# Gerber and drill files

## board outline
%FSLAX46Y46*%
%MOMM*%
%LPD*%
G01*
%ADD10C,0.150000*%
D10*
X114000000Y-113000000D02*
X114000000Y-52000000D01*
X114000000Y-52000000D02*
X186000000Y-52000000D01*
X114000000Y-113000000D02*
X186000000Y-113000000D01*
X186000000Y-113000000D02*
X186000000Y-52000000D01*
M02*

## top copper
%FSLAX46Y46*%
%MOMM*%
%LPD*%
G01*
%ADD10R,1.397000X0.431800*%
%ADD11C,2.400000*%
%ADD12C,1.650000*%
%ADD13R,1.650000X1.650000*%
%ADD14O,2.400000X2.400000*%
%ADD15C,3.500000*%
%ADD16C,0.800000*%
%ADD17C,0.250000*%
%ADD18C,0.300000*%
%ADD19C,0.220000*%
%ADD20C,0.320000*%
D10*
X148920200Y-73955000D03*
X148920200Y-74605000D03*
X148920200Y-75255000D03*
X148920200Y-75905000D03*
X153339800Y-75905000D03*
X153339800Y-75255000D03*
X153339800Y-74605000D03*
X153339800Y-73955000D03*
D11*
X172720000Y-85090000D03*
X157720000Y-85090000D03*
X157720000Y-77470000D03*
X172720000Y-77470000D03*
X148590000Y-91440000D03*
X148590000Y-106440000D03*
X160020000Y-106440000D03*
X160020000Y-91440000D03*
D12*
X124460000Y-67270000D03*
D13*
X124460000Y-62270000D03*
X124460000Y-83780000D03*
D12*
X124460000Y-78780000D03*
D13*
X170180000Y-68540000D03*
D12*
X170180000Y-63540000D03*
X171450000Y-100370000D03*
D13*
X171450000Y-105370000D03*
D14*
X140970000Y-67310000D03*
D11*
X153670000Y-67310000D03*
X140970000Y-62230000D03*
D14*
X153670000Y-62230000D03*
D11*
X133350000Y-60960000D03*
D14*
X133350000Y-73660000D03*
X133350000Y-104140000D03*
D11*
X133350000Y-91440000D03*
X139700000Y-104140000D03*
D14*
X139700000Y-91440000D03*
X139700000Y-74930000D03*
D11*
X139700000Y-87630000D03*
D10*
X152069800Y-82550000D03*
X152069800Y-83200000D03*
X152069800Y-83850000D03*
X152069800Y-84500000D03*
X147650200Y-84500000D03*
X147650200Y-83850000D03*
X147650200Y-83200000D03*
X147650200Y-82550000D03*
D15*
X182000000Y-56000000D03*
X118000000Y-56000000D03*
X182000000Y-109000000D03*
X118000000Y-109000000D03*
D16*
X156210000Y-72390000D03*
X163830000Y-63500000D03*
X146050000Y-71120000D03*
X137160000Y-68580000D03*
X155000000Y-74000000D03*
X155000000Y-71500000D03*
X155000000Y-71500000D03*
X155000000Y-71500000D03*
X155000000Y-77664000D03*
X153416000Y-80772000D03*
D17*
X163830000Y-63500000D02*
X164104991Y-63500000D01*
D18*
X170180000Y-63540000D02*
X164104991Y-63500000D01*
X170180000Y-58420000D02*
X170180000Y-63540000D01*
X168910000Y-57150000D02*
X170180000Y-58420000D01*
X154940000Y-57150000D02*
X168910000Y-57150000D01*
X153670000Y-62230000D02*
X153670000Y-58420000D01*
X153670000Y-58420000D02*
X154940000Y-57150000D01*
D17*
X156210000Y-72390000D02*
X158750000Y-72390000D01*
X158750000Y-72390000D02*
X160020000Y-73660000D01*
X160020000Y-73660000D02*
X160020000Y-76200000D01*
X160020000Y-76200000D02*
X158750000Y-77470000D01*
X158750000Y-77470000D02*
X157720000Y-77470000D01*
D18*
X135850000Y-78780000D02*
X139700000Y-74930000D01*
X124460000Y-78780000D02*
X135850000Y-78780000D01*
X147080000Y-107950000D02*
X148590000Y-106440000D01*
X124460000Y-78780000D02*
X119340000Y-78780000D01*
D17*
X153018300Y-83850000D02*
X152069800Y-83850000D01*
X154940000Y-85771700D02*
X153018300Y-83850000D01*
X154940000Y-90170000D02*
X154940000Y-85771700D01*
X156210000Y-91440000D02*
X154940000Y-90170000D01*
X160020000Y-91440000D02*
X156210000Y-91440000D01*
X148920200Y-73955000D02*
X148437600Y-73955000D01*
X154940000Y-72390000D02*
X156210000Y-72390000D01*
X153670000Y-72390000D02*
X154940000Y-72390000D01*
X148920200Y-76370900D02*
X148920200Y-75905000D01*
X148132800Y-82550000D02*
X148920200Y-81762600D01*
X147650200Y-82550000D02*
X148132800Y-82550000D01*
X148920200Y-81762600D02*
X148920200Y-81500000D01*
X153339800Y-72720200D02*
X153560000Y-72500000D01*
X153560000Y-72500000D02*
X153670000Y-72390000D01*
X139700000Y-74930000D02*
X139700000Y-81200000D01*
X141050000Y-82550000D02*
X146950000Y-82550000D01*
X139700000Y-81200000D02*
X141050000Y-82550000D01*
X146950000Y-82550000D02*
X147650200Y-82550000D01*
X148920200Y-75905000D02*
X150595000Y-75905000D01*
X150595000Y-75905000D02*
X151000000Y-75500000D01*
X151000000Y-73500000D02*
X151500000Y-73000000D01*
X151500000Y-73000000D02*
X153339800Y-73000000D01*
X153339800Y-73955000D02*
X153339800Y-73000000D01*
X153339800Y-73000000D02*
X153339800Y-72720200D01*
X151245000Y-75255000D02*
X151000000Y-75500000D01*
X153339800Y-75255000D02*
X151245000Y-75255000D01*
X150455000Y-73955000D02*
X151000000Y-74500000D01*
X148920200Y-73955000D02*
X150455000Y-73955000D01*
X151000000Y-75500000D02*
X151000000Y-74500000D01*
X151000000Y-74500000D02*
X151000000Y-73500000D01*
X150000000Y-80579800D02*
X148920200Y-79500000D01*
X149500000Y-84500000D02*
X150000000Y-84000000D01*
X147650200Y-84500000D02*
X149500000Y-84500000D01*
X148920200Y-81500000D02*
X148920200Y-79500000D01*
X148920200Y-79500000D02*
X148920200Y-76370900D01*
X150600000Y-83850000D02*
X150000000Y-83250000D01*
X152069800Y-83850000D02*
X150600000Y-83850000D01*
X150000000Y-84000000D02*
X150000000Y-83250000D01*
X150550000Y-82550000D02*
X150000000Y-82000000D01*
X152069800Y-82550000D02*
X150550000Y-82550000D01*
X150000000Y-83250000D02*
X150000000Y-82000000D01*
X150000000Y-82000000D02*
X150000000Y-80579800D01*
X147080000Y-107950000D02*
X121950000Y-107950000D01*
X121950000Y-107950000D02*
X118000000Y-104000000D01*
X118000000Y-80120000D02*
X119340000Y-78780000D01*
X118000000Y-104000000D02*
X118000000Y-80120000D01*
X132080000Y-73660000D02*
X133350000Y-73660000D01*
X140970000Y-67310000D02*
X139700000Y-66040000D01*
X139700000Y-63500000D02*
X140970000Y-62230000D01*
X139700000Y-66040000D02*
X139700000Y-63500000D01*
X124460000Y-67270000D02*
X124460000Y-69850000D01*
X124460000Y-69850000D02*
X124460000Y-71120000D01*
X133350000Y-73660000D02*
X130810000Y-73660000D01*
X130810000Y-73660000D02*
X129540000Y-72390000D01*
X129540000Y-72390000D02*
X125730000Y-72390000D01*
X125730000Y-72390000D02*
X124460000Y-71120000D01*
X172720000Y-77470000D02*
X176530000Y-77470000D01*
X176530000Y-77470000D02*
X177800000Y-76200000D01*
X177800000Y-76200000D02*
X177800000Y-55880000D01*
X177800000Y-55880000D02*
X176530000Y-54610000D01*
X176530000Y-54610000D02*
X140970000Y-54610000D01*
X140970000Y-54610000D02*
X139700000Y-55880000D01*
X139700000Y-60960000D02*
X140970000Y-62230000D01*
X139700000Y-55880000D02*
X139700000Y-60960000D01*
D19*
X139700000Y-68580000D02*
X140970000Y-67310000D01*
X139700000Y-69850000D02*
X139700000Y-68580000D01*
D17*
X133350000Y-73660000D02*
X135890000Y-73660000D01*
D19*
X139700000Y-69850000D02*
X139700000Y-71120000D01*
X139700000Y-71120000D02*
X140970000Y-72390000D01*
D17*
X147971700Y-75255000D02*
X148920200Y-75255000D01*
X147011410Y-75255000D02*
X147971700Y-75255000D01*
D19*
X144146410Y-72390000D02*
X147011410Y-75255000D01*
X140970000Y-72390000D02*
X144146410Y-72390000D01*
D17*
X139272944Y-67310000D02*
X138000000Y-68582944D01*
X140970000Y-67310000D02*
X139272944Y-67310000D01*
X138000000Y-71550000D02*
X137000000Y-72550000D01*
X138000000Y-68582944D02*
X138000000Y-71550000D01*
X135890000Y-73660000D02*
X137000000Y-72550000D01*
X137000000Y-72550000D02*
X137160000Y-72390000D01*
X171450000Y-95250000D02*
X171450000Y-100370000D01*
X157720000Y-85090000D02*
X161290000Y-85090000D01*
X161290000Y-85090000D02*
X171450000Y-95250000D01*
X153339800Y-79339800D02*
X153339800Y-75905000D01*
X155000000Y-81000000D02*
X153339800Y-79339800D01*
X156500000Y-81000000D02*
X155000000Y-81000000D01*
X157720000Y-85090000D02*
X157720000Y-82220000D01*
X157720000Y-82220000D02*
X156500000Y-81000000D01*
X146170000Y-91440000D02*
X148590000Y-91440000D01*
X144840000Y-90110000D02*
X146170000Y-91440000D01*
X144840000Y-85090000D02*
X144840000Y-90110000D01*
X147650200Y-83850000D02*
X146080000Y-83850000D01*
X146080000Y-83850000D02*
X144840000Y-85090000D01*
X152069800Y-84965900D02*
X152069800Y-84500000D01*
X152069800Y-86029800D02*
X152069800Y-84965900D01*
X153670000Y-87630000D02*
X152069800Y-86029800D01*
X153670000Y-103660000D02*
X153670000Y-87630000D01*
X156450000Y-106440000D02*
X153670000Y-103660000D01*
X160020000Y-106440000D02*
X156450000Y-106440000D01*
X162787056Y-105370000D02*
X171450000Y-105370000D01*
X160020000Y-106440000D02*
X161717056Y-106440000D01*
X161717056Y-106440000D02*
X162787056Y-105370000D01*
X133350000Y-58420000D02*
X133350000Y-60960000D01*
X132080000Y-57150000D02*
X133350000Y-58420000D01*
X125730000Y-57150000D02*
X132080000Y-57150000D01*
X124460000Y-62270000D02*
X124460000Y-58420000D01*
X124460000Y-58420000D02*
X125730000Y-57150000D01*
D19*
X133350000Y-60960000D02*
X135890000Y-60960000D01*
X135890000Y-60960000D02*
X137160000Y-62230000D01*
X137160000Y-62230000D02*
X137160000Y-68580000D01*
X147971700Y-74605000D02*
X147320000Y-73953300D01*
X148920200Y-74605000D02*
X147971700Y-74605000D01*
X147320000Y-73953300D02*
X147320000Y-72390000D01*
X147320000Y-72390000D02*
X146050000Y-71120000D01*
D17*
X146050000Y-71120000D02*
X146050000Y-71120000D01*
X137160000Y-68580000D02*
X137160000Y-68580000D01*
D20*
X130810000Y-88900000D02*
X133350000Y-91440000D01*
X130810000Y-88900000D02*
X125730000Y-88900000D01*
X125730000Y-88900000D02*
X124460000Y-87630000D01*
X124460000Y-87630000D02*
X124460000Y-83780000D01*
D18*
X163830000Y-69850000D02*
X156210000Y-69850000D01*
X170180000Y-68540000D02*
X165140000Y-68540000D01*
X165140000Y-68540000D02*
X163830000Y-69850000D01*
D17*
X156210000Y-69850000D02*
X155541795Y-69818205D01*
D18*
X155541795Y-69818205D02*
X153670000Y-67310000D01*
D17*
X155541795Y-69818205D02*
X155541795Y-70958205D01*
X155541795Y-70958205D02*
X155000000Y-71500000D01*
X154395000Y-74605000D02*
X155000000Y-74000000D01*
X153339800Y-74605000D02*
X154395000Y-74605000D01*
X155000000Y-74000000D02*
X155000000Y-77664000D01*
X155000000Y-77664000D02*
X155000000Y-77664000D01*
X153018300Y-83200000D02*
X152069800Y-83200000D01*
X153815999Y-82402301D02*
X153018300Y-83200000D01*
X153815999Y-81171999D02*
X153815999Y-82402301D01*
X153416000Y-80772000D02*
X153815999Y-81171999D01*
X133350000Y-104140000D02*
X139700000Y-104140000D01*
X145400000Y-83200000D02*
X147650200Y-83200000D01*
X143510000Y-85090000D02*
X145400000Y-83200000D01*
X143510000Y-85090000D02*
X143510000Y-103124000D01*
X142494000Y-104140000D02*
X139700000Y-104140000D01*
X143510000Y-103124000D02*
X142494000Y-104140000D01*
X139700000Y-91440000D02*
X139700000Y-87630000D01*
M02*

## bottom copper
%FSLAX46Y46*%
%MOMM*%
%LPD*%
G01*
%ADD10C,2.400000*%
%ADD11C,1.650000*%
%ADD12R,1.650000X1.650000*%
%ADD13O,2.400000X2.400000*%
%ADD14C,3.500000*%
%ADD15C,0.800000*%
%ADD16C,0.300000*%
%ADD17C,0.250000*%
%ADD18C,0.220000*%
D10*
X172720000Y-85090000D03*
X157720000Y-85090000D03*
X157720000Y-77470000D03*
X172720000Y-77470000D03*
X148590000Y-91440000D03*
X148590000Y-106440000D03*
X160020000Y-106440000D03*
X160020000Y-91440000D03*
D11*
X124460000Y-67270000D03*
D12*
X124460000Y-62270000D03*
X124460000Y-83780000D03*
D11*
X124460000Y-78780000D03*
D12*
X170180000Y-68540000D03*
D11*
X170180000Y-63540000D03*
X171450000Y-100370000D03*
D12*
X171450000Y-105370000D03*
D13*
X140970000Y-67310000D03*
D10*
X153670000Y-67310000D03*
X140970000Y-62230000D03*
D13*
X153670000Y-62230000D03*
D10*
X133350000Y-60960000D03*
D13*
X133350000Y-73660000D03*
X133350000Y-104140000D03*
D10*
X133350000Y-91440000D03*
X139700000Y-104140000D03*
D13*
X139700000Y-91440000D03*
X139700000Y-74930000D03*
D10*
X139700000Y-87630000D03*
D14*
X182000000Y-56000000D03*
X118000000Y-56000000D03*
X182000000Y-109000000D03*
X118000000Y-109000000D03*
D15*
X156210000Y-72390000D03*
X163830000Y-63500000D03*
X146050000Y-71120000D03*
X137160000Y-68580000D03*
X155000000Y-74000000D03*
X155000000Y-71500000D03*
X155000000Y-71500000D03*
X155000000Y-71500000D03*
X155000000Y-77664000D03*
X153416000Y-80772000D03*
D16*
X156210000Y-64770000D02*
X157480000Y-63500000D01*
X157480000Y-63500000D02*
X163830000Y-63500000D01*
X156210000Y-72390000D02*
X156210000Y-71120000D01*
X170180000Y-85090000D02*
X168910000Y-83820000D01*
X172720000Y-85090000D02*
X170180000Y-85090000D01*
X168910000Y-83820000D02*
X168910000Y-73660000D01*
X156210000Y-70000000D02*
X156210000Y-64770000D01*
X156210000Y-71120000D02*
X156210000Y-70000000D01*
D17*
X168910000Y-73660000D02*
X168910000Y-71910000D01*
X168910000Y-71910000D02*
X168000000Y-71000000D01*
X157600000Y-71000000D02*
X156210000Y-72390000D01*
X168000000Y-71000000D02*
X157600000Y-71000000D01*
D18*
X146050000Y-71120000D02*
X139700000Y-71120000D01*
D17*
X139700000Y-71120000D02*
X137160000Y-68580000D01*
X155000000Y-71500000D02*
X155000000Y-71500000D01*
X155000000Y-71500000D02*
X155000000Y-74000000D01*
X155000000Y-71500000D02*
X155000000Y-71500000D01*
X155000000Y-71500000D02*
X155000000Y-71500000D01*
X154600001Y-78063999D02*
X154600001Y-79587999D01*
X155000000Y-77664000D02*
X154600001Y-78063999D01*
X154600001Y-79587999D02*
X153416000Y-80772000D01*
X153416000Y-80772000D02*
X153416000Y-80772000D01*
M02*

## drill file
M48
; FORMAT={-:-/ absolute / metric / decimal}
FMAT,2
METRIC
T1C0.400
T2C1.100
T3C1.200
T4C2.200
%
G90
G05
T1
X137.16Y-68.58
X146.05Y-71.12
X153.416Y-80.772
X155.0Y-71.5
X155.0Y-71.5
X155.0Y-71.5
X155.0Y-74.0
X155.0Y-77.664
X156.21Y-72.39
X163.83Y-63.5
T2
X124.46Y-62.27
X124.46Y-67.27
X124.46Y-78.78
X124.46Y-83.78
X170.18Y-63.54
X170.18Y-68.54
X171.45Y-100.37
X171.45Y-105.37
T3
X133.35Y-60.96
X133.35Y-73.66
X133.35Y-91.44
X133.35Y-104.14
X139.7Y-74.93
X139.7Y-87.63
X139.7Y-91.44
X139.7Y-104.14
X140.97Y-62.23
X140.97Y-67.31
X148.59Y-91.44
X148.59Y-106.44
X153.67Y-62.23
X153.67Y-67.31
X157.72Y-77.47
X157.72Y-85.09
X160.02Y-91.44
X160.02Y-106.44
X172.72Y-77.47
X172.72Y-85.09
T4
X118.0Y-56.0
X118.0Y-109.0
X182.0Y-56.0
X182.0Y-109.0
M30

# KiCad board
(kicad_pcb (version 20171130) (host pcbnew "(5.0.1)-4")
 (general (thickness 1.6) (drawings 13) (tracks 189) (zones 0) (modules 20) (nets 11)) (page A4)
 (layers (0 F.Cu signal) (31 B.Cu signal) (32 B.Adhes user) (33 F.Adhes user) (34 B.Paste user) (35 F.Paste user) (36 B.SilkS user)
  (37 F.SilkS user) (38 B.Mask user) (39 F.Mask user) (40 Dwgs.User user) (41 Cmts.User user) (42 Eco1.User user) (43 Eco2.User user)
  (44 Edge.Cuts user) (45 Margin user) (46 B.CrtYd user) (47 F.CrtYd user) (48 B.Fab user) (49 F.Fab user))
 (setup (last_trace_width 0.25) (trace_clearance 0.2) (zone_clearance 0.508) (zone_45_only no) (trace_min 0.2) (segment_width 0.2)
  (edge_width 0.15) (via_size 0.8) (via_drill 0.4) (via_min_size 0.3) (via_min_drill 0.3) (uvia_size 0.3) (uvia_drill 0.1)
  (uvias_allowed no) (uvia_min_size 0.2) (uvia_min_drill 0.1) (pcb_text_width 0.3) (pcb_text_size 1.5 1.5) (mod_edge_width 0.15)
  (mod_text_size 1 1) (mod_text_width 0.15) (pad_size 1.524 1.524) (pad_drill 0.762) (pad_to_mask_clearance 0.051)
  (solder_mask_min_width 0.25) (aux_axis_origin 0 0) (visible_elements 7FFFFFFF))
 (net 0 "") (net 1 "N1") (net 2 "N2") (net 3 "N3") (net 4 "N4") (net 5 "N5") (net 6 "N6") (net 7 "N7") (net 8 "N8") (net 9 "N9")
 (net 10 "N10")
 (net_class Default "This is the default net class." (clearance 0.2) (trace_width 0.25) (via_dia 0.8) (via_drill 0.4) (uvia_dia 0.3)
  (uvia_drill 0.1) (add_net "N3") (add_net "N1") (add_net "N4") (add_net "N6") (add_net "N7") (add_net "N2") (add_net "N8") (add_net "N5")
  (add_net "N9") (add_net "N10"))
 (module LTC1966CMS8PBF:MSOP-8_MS (layer F.Cu) (at 151.13 74.93)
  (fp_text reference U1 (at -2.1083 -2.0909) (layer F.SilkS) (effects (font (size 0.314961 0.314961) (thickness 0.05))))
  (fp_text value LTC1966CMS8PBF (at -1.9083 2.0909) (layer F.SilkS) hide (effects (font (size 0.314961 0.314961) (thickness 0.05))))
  (pad 1 smd rect (at -2.2098 -0.975) (size 1.397 0.4318) (layers F.Cu F.Paste F.Mask) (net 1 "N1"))
  (pad 2 smd rect (at -2.2098 -0.325) (size 1.397 0.4318) (layers F.Cu F.Paste F.Mask) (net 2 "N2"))
  (pad 3 smd rect (at -2.2098 0.325) (size 1.397 0.4318) (layers F.Cu F.Paste F.Mask) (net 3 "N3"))
  (pad 4 smd rect (at -2.2098 0.975) (size 1.397 0.4318) (layers F.Cu F.Paste F.Mask) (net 1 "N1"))
  (pad 5 smd rect (at 2.2098 0.975) (size 1.397 0.4318) (layers F.Cu F.Paste F.Mask) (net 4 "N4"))
  (pad 6 smd rect (at 2.2098 0.325) (size 1.397 0.4318) (layers F.Cu F.Paste F.Mask) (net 1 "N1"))
  (pad 7 smd rect (at 2.2098 -0.325) (size 1.397 0.4318) (layers F.Cu F.Paste F.Mask) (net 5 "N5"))
  (pad 8 smd rect (at 2.2098 -0.975) (size 1.397 0.4318) (layers F.Cu F.Paste F.Mask) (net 1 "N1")))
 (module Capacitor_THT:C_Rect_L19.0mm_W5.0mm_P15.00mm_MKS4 (layer F.Cu) (at 172.72 85.09 180)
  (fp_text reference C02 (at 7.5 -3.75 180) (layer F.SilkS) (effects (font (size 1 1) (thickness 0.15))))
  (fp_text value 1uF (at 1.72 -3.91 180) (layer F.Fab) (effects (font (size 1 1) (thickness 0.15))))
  (pad 1 thru_hole circle (at 0 0 180) (size 2.4 2.4) (drill 1.2) (layers *.Cu *.Mask) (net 1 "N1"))
  (pad 2 thru_hole circle (at 15 0 180) (size 2.4 2.4) (drill 1.2) (layers *.Cu *.Mask) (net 4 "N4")))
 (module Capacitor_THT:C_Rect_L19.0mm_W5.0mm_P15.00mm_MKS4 (layer F.Cu) (at 172.72 77.47 180)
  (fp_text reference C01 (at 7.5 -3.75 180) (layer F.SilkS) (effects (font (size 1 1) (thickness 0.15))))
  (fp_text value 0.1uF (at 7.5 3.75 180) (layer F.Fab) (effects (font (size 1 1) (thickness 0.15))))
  (pad 2 thru_hole circle (at 15 0 180) (size 2.4 2.4) (drill 1.2) (layers *.Cu *.Mask) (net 1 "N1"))
  (pad 1 thru_hole circle (at 0 0 180) (size 2.4 2.4) (drill 1.2) (layers *.Cu *.Mask) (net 3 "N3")))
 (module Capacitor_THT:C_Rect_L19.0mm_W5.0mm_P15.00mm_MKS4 (layer F.Cu) (at 148.59 91.44 270)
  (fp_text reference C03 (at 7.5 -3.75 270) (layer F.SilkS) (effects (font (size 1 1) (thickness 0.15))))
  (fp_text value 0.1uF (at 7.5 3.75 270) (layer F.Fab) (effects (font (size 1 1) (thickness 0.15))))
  (pad 1 thru_hole circle (at 0 0 270) (size 2.4 2.4) (drill 1.2) (layers *.Cu *.Mask) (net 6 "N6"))
  (pad 2 thru_hole circle (at 15 0 270) (size 2.4 2.4) (drill 1.2) (layers *.Cu *.Mask) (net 1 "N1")))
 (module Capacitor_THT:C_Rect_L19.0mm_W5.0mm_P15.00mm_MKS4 (layer F.Cu) (at 160.02 91.44 270)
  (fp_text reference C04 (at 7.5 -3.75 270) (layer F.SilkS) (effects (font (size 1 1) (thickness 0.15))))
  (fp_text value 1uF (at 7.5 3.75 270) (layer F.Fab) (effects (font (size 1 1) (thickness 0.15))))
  (pad 2 thru_hole circle (at 15 0 270) (size 2.4 2.4) (drill 1.2) (layers *.Cu *.Mask) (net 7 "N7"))
  (pad 1 thru_hole circle (at 0 0 270) (size 2.4 2.4) (drill 1.2) (layers *.Cu *.Mask) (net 1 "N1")))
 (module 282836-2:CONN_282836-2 (layer F.Cu) (at 124.46 64.77 270)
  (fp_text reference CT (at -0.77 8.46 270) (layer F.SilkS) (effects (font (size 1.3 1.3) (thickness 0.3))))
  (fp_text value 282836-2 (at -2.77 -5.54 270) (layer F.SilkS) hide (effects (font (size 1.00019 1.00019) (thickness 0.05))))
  (pad 2 thru_hole circle (at 2.5 0 270) (size 1.65 1.65) (drill 1.1) (layers *.Cu *.Mask) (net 3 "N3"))
  (pad 1 thru_hole rect (at -2.5 0 270) (size 1.65 1.65) (drill 1.1) (layers *.Cu *.Mask) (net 2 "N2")))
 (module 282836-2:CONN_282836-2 (layer F.Cu) (at 124.46 81.28 90)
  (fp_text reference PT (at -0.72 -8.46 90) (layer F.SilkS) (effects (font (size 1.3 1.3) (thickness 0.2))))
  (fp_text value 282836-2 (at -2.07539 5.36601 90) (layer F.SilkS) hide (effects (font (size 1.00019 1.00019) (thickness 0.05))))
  (pad 1 thru_hole rect (at -2.5 0 90) (size 1.65 1.65) (drill 1.1) (layers *.Cu *.Mask) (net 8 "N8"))
  (pad 2 thru_hole circle (at 2.5 0 90) (size 1.65 1.65) (drill 1.1) (layers *.Cu *.Mask) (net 1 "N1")))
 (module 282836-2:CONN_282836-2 (layer F.Cu) (at 170.18 66.04 90)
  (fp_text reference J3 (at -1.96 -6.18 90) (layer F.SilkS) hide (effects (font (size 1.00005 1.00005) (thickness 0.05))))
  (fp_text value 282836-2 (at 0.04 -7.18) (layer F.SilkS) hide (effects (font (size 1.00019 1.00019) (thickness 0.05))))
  (pad 1 thru_hole rect (at -2.5 0 90) (size 1.65 1.65) (drill 1.1) (layers *.Cu *.Mask) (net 5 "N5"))
  (pad 2 thru_hole circle (at 2.5 0 90) (size 1.65 1.65) (drill 1.1) (layers *.Cu *.Mask) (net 1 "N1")))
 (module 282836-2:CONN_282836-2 (layer F.Cu) (at 171.45 102.87 90)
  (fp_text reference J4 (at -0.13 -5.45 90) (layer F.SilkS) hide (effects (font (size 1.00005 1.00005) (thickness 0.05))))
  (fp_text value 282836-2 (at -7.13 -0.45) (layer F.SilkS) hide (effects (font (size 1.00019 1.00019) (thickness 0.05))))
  (pad 2 thru_hole circle (at 2.5 0 90) (size 1.65 1.65) (drill 1.1) (layers *.Cu *.Mask) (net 4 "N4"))
  (pad 1 thru_hole rect (at -2.5 0 90) (size 1.65 1.65) (drill 1.1) (layers *.Cu *.Mask) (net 7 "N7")))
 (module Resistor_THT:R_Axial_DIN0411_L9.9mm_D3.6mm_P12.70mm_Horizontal (layer F.Cu) (at 153.67 67.31 180)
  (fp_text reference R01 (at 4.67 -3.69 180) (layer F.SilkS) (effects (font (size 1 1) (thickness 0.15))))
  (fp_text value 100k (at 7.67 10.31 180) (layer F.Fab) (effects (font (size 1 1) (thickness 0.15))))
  (pad 2 thru_hole oval (at 12.7 0 180) (size 2.4 2.4) (drill 1.2) (layers *.Cu *.Mask) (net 3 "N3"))
  (pad 1 thru_hole circle (at 0 0 180) (size 2.4 2.4) (drill 1.2) (layers *.Cu *.Mask) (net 5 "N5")))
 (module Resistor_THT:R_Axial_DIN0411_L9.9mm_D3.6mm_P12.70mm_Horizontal (layer F.Cu) (at 140.97 62.23)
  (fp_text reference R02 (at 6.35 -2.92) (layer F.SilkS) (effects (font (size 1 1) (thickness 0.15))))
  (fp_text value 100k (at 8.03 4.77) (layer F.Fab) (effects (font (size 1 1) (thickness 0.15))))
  (pad 1 thru_hole circle (at 0 0) (size 2.4 2.4) (drill 1.2) (layers *.Cu *.Mask) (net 3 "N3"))
  (pad 2 thru_hole oval (at 12.7 0) (size 2.4 2.4) (drill 1.2) (layers *.Cu *.Mask) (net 1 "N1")))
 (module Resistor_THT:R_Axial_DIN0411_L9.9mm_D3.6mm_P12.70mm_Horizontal (layer F.Cu) (at 133.35 60.96 270)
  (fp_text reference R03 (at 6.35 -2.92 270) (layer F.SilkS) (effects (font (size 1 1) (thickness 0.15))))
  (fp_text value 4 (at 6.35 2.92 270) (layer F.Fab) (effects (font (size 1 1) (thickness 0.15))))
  (pad 1 thru_hole circle (at 0 0 270) (size 2.4 2.4) (drill 1.2) (layers *.Cu *.Mask) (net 2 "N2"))
  (pad 2 thru_hole oval (at 12.7 0 270) (size 2.4 2.4) (drill 1.2) (layers *.Cu *.Mask) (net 3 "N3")))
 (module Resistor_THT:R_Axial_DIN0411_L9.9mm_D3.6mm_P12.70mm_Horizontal (layer F.Cu) (at 133.35 91.44 270)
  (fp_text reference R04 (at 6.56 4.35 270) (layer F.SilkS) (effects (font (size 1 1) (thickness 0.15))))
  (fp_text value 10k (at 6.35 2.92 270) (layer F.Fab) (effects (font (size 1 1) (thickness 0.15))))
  (pad 2 thru_hole oval (at 12.7 0 270) (size 2.4 2.4) (drill 1.2) (layers *.Cu *.Mask) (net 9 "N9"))
  (pad 1 thru_hole circle (at 0 0 270) (size 2.4 2.4) (drill 1.2) (layers *.Cu *.Mask) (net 8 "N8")))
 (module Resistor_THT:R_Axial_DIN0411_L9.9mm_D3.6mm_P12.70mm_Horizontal (layer F.Cu) (at 139.7 104.14 90)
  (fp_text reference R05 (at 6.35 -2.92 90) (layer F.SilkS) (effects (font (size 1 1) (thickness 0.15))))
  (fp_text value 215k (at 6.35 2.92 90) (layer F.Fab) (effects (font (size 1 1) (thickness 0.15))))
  (pad 1 thru_hole circle (at 0 0 90) (size 2.4 2.4) (drill 1.2) (layers *.Cu *.Mask) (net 9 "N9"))
  (pad 2 thru_hole oval (at 12.7 0 90) (size 2.4 2.4) (drill 1.2) (layers *.Cu *.Mask) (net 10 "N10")))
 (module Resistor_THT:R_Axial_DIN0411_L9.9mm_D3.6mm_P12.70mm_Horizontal (layer F.Cu) (at 139.7 87.63 90)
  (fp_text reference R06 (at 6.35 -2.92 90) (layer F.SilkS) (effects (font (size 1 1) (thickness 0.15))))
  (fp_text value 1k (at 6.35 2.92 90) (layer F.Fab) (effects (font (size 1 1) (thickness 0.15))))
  (pad 2 thru_hole oval (at 12.7 0 90) (size 2.4 2.4) (drill 1.2) (layers *.Cu *.Mask) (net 1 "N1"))
  (pad 1 thru_hole circle (at 0 0 90) (size 2.4 2.4) (drill 1.2) (layers *.Cu *.Mask) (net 10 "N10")))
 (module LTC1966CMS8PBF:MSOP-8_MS (layer F.Cu) (at 149.86 83.525)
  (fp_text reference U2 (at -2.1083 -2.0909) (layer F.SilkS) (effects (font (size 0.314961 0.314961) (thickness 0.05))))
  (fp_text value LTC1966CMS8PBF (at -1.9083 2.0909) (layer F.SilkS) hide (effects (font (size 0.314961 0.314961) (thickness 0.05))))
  (pad 8 smd rect (at 2.2098 -0.975) (size 1.397 0.4318) (layers F.Cu F.Paste F.Mask) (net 1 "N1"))
  (pad 7 smd rect (at 2.2098 -0.325) (size 1.397 0.4318) (layers F.Cu F.Paste F.Mask) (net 5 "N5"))
  (pad 6 smd rect (at 2.2098 0.325) (size 1.397 0.4318) (layers F.Cu F.Paste F.Mask) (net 1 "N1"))
  (pad 5 smd rect (at 2.2098 0.975) (size 1.397 0.4318) (layers F.Cu F.Paste F.Mask) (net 7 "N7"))
  (pad 4 smd rect (at -2.2098 0.975) (size 1.397 0.4318) (layers F.Cu F.Paste F.Mask) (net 1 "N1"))
  (pad 3 smd rect (at -2.2098 0.325) (size 1.397 0.4318) (layers F.Cu F.Paste F.Mask) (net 6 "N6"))
  (pad 2 smd rect (at -2.2098 -0.325) (size 1.397 0.4318) (layers F.Cu F.Paste F.Mask) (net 9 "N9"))
  (pad 1 smd rect (at -2.2098 -0.975) (size 1.397 0.4318) (layers F.Cu F.Paste F.Mask) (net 1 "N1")))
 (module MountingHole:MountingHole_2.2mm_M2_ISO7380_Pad (layer F.Cu) (at 182 56)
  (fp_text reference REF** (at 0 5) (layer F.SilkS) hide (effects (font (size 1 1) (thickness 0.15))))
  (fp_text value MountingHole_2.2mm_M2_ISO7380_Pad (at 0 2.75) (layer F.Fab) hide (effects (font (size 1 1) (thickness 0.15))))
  (pad 1 thru_hole circle (at 0 0) (size 3.5 3.5) (drill 2.2) (layers *.Cu *.Mask)))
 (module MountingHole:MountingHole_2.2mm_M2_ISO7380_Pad (layer F.Cu) (at 118 56)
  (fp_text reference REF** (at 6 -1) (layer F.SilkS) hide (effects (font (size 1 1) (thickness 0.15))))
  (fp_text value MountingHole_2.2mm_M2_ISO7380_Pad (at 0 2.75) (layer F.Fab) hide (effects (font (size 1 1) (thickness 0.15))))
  (pad 1 thru_hole circle (at 0 0) (size 3.5 3.5) (drill 2.2) (layers *.Cu *.Mask)))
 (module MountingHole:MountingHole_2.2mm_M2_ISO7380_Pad (layer F.Cu) (at 182 109)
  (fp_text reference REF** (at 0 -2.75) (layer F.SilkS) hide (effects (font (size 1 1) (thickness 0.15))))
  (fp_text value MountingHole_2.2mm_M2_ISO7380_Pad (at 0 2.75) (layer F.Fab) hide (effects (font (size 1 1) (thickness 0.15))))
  (pad 1 thru_hole circle (at 0 0) (size 3.5 3.5) (drill 2.2) (layers *.Cu *.Mask)))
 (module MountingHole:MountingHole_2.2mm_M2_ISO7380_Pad (layer F.Cu) (at 118 109)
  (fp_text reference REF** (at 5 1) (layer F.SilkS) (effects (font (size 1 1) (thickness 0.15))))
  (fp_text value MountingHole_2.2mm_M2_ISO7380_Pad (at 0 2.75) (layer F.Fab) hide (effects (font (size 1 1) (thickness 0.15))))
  (pad 1 thru_hole circle (at 0 0) (size 3.5 3.5) (drill 2.2) (layers *.Cu *.Mask)))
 (gr_line (start 114 113) (end 114 52) (layer Edge.Cuts) (width 0.15))
 (gr_line (start 114 52) (end 186 52) (layer Edge.Cuts) (width 0.15))
 (gr_line (start 114 113) (end 186 113) (layer Edge.Cuts) (width 0.15))
 (gr_line (start 186 113) (end 186 52) (layer Edge.Cuts) (width 0.15))
 (via (at 156.21 72.39) (size 0.8) (drill 0.4) (layers F.Cu B.Cu) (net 1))
 (via (at 163.83 63.5) (size 0.8) (drill 0.4) (layers F.Cu B.Cu) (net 1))
 (segment (start 163.83 63.5) (end 164.104991 63.5) (width 0.25) (layer F.Cu) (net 1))
 (segment (start 170.18 63.54) (end 164.104991 63.5) (width 0.3) (layer F.Cu) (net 1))
 (segment (start 170.18 58.42) (end 170.18 63.54) (width 0.3) (layer F.Cu) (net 1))
 (segment (start 168.91 57.15) (end 170.18 58.42) (width 0.3) (layer F.Cu) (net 1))
 (segment (start 154.94 57.15) (end 168.91 57.15) (width 0.3) (layer F.Cu) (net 1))
 (segment (start 153.67 62.23) (end 153.67 58.42) (width 0.3) (layer F.Cu) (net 1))
 (segment (start 153.67 58.42) (end 154.94 57.15) (width 0.3) (layer F.Cu) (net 1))
 (segment (start 156.21 64.77) (end 157.48 63.5) (width 0.3) (layer B.Cu) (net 1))
 (segment (start 157.48 63.5) (end 163.83 63.5) (width 0.3) (layer B.Cu) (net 1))
 (segment (start 156.21 72.39) (end 158.75 72.39) (width 0.25) (layer F.Cu) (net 1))
 (segment (start 158.75 72.39) (end 160.02 73.66) (width 0.25) (layer F.Cu) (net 1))
 (segment (start 160.02 73.66) (end 160.02 76.2) (width 0.25) (layer F.Cu) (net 1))
 (segment (start 160.02 76.2) (end 158.75 77.47) (width 0.25) (layer F.Cu) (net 1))
 (segment (start 158.75 77.47) (end 157.72 77.47) (width 0.25) (layer F.Cu) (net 1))
 (segment (start 156.21 72.39) (end 156.21 71.12) (width 0.3) (layer B.Cu) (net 1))
 (segment (start 170.18 85.09) (end 168.91 83.82) (width 0.3) (layer B.Cu) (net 1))
 (segment (start 172.72 85.09) (end 170.18 85.09) (width 0.3) (layer B.Cu) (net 1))
 (segment (start 168.91 83.82) (end 168.91 73.66) (width 0.3) (layer B.Cu) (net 1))
 (segment (start 135.85 78.78) (end 139.7 74.93) (width 0.3) (layer F.Cu) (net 1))
 (segment (start 124.46 78.78) (end 135.85 78.78) (width 0.3) (layer F.Cu) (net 1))
 (segment (start 147.08 107.95) (end 148.59 106.44) (width 0.3) (layer F.Cu) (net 1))
 (segment (start 124.46 78.78) (end 119.34 78.78) (width 0.3) (layer F.Cu) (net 1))
 (segment (start 153.0183 83.85) (end 152.0698 83.85) (width 0.25) (layer F.Cu) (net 1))
 (segment (start 154.94 85.7717) (end 153.0183 83.85) (width 0.25) (layer F.Cu) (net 1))
 (segment (start 154.94 90.17) (end 154.94 85.7717) (width 0.25) (layer F.Cu) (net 1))
 (segment (start 156.21 91.44) (end 154.94 90.17) (width 0.25) (layer F.Cu) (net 1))
 (segment (start 160.02 91.44) (end 156.21 91.44) (width 0.25) (layer F.Cu) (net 1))
 (segment (start 148.9202 73.955) (end 148.4376 73.955) (width 0.25) (layer F.Cu) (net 1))
 (segment (start 154.94 72.39) (end 156.21 72.39) (width 0.25) (layer F.Cu) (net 1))
 (segment (start 153.67 72.39) (end 154.94 72.39) (width 0.25) (layer F.Cu) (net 1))
 (segment (start 148.9202 76.3709) (end 148.9202 75.905) (width 0.25) (layer F.Cu) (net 1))
 (segment (start 148.1328 82.55) (end 148.9202 81.7626) (width 0.25) (layer F.Cu) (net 1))
 (segment (start 147.6502 82.55) (end 148.1328 82.55) (width 0.25) (layer F.Cu) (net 1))
 (segment (start 148.9202 81.7626) (end 148.9202 81.5) (width 0.25) (layer F.Cu) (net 1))
 (segment (start 153.3398 72.7202) (end 153.56 72.5) (width 0.25) (layer F.Cu) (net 1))
 (segment (start 153.56 72.5) (end 153.67 72.39) (width 0.25) (layer F.Cu) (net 1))
 (segment (start 156.21 70) (end 156.21 64.77) (width 0.3) (layer B.Cu) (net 1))
 (segment (start 156.21 71.12) (end 156.21 70) (width 0.3) (layer B.Cu) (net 1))
 (segment (start 139.7 74.93) (end 139.7 81.2) (width 0.25) (layer F.Cu) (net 1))
 (segment (start 141.05 82.55) (end 146.95 82.55) (width 0.25) (layer F.Cu) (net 1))
 (segment (start 139.7 81.2) (end 141.05 82.55) (width 0.25) (layer F.Cu) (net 1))
 (segment (start 146.95 82.55) (end 147.6502 82.55) (width 0.25) (layer F.Cu) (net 1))
 (segment (start 148.9202 75.905) (end 150.595 75.905) (width 0.25) (layer F.Cu) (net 1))
 (segment (start 150.595 75.905) (end 151 75.5) (width 0.25) (layer F.Cu) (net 1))
 (segment (start 151 73.5) (end 151.5 73) (width 0.25) (layer F.Cu) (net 1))
 (segment (start 151.5 73) (end 153.3398 73) (width 0.25) (layer F.Cu) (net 1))
 (segment (start 153.3398 73.955) (end 153.3398 73) (width 0.25) (layer F.Cu) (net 1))
 (segment (start 153.3398 73) (end 153.3398 72.7202) (width 0.25) (layer F.Cu) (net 1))
 (segment (start 151.245 75.255) (end 151 75.5) (width 0.25) (layer F.Cu) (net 1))
 (segment (start 153.3398 75.255) (end 151.245 75.255) (width 0.25) (layer F.Cu) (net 1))
 (segment (start 150.455 73.955) (end 151 74.5) (width 0.25) (layer F.Cu) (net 1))
 (segment (start 148.9202 73.955) (end 150.455 73.955) (width 0.25) (layer F.Cu) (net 1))
 (segment (start 151 75.5) (end 151 74.5) (width 0.25) (layer F.Cu) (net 1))
 (segment (start 151 74.5) (end 151 73.5) (width 0.25) (layer F.Cu) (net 1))
 (segment (start 150 80.5798) (end 148.9202 79.5) (width 0.25) (layer F.Cu) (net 1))
 (segment (start 149.5 84.5) (end 150 84) (width 0.25) (layer F.Cu) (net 1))
 (segment (start 147.6502 84.5) (end 149.5 84.5) (width 0.25) (layer F.Cu) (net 1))
 (segment (start 148.9202 81.5) (end 148.9202 79.5) (width 0.25) (layer F.Cu) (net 1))
 (segment (start 148.9202 79.5) (end 148.9202 76.3709) (width 0.25) (layer F.Cu) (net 1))
 (segment (start 150.6 83.85) (end 150 83.25) (width 0.25) (layer F.Cu) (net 1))
 (segment (start 152.0698 83.85) (end 150.6 83.85) (width 0.25) (layer F.Cu) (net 1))
 (segment (start 150 84) (end 150 83.25) (width 0.25) (layer F.Cu) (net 1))
 (segment (start 150.55 82.55) (end 150 82) (width 0.25) (layer F.Cu) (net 1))
 (segment (start 152.0698 82.55) (end 150.55 82.55) (width 0.25) (layer F.Cu) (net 1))
 (segment (start 150 83.25) (end 150 82) (width 0.25) (layer F.Cu) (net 1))
 (segment (start 150 82) (end 150 80.5798) (width 0.25) (layer F.Cu) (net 1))
 (segment (start 147.08 107.95) (end 121.95 107.95) (width 0.25) (layer F.Cu) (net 1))
 (segment (start 121.95 107.95) (end 118 104) (width 0.25) (layer F.Cu) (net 1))
 (segment (start 118 80.12) (end 119.34 78.78) (width 0.25) (layer F.Cu) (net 1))
 (segment (start 118 104) (end 118 80.12) (width 0.25) (layer F.Cu) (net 1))
 (segment (start 168.91 73.66) (end 168.91 71.91) (width 0.25) (layer B.Cu) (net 1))
 (segment (start 168.91 71.91) (end 168 71) (width 0.25) (layer B.Cu) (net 1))
 (segment (start 157.6 71) (end 156.21 72.39) (width 0.25) (layer B.Cu) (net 1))
 (segment (start 168 71) (end 157.6 71) (width 0.25) (layer B.Cu) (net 1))
 (segment (start 132.08 73.66) (end 133.35 73.66) (width 0.25) (layer F.Cu) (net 3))
 (segment (start 140.97 67.31) (end 139.7 66.04) (width 0.25) (layer F.Cu) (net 3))
 (segment (start 139.7 63.5) (end 140.97 62.23) (width 0.25) (layer F.Cu) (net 3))
 (segment (start 139.7 66.04) (end 139.7 63.5) (width 0.25) (layer F.Cu) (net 3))
 (segment (start 124.46 67.27) (end 124.46 69.85) (width 0.25) (layer F.Cu) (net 3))
 (segment (start 124.46 69.85) (end 124.46 71.12) (width 0.25) (layer F.Cu) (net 3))
 (segment (start 133.35 73.66) (end 130.81 73.66) (width 0.25) (layer F.Cu) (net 3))
 (segment (start 130.81 73.66) (end 129.54 72.39) (width 0.25) (layer F.Cu) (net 3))
 (segment (start 129.54 72.39) (end 125.73 72.39) (width 0.25) (layer F.Cu) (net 3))
 (segment (start 125.73 72.39) (end 124.46 71.12) (width 0.25) (layer F.Cu) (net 3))
 (segment (start 172.72 77.47) (end 176.53 77.47) (width 0.25) (layer F.Cu) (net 3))
 (segment (start 176.53 77.47) (end 177.8 76.2) (width 0.25) (layer F.Cu) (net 3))
 (segment (start 177.8 76.2) (end 177.8 55.88) (width 0.25) (layer F.Cu) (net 3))
 (segment (start 177.8 55.88) (end 176.53 54.61) (width 0.25) (layer F.Cu) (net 3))
 (segment (start 176.53 54.61) (end 140.97 54.61) (width 0.25) (layer F.Cu) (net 3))
 (segment (start 140.97 54.61) (end 139.7 55.88) (width 0.25) (layer F.Cu) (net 3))
 (segment (start 139.7 60.96) (end 140.97 62.23) (width 0.25) (layer F.Cu) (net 3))
 (segment (start 139.7 55.88) (end 139.7 60.96) (width 0.25) (layer F.Cu) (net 3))
 (segment (start 139.7 68.58) (end 140.97 67.31) (width 0.22) (layer F.Cu) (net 3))
 (segment (start 139.7 69.85) (end 139.7 68.58) (width 0.22) (layer F.Cu) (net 3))
 (segment (start 133.35 73.66) (end 135.89 73.66) (width 0.25) (layer F.Cu) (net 3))
 (segment (start 139.7 69.85) (end 139.7 71.12) (width 0.22) (layer F.Cu) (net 3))
 (segment (start 139.7 71.12) (end 140.97 72.39) (width 0.22) (layer F.Cu) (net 3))
 (segment (start 147.9717 75.255) (end 148.9202 75.255) (width 0.25) (layer F.Cu) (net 3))
 (segment (start 147.01141 75.255) (end 147.9717 75.255) (width 0.25) (layer F.Cu) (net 3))
 (segment (start 144.14641 72.39) (end 147.01141 75.255) (width 0.22) (layer F.Cu) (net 3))
 (segment (start 140.97 72.39) (end 144.14641 72.39) (width 0.22) (layer F.Cu) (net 3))
 (segment (start 139.272944 67.31) (end 138 68.582944) (width 0.25) (layer F.Cu) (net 3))
 (segment (start 140.97 67.31) (end 139.272944 67.31) (width 0.25) (layer F.Cu) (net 3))
 (segment (start 138 71.55) (end 137 72.55) (width 0.25) (layer F.Cu) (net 3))
 (segment (start 138 68.582944) (end 138 71.55) (width 0.25) (layer F.Cu) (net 3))
 (segment (start 135.89 73.66) (end 137 72.55) (width 0.25) (layer F.Cu) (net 3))
 (segment (start 137 72.55) (end 137.16 72.39) (width 0.25) (layer F.Cu) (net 3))
 (segment (start 171.45 95.25) (end 171.45 100.37) (width 0.25) (layer F.Cu) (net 4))
 (segment (start 157.72 85.09) (end 161.29 85.09) (width 0.25) (layer F.Cu) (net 4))
 (segment (start 161.29 85.09) (end 171.45 95.25) (width 0.25) (layer F.Cu) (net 4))
 (segment (start 153.3398 79.3398) (end 153.3398 75.905) (width 0.25) (layer F.Cu) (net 4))
 (segment (start 155 81) (end 153.3398 79.3398) (width 0.25) (layer F.Cu) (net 4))
 (segment (start 156.5 81) (end 155 81) (width 0.25) (layer F.Cu) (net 4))
 (segment (start 157.72 85.09) (end 157.72 82.22) (width 0.25) (layer F.Cu) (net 4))
 (segment (start 157.72 82.22) (end 156.5 81) (width 0.25) (layer F.Cu) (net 4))
 (segment (start 146.17 91.44) (end 148.59 91.44) (width 0.25) (layer F.Cu) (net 6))
 (segment (start 144.84 90.11) (end 146.17 91.44) (width 0.25) (layer F.Cu) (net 6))
 (segment (start 144.84 85.09) (end 144.84 90.11) (width 0.25) (layer F.Cu) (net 6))
 (segment (start 147.6502 83.85) (end 146.08 83.85) (width 0.25) (layer F.Cu) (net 6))
 (segment (start 146.08 83.85) (end 144.84 85.09) (width 0.25) (layer F.Cu) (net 6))
 (segment (start 152.0698 84.9659) (end 152.0698 84.5) (width 0.25) (layer F.Cu) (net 7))
 (segment (start 152.0698 86.0298) (end 152.0698 84.9659) (width 0.25) (layer F.Cu) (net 7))
 (segment (start 153.67 87.63) (end 152.0698 86.0298) (width 0.25) (layer F.Cu) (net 7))
 (segment (start 153.67 103.66) (end 153.67 87.63) (width 0.25) (layer F.Cu) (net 7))
 (segment (start 156.45 106.44) (end 153.67 103.66) (width 0.25) (layer F.Cu) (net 7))
 (segment (start 160.02 106.44) (end 156.45 106.44) (width 0.25) (layer F.Cu) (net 7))
 (segment (start 162.787056 105.37) (end 171.45 105.37) (width 0.25) (layer F.Cu) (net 7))
 (segment (start 160.02 106.44) (end 161.717056 106.44) (width 0.25) (layer F.Cu) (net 7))
 (segment (start 161.717056 106.44) (end 162.787056 105.37) (width 0.25) (layer F.Cu) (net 7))
 (segment (start 133.35 58.42) (end 133.35 60.96) (width 0.25) (layer F.Cu) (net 2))
 (segment (start 132.08 57.15) (end 133.35 58.42) (width 0.25) (layer F.Cu) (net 2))
 (segment (start 125.73 57.15) (end 132.08 57.15) (width 0.25) (layer F.Cu) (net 2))
 (segment (start 124.46 62.27) (end 124.46 58.42) (width 0.25) (layer F.Cu) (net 2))
 (segment (start 124.46 58.42) (end 125.73 57.15) (width 0.25) (layer F.Cu) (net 2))
 (segment (start 133.35 60.96) (end 135.89 60.96) (width 0.22) (layer F.Cu) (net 2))
 (segment (start 135.89 60.96) (end 137.16 62.23) (width 0.22) (layer F.Cu) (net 2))
 (segment (start 137.16 62.23) (end 137.16 68.58) (width 0.22) (layer F.Cu) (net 2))
 (segment (start 147.9717 74.605) (end 147.32 73.9533) (width 0.22) (layer F.Cu) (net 2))
 (segment (start 148.9202 74.605) (end 147.9717 74.605) (width 0.22) (layer F.Cu) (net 2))
 (segment (start 147.32 73.9533) (end 147.32 72.39) (width 0.22) (layer F.Cu) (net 2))
 (segment (start 147.32 72.39) (end 146.05 71.12) (width 0.22) (layer F.Cu) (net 2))
 (segment (start 146.05 71.12) (end 146.05 71.12) (width 0.25) (layer F.Cu) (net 2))
 (via (at 146.05 71.12) (size 0.8) (drill 0.4) (layers F.Cu B.Cu) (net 2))
 (segment (start 137.16 68.58) (end 137.16 68.58) (width 0.25) (layer F.Cu) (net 2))
 (via (at 137.16 68.58) (size 0.8) (drill 0.4) (layers F.Cu B.Cu) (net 2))
 (segment (start 146.05 71.12) (end 139.7 71.12) (width 0.22) (layer B.Cu) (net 2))
 (segment (start 139.7 71.12) (end 137.16 68.58) (width 0.25) (layer B.Cu) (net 2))
 (segment (start 130.81 88.9) (end 133.35 91.44) (width 0.32) (layer F.Cu) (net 8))
 (segment (start 130.81 88.9) (end 125.73 88.9) (width 0.32) (layer F.Cu) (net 8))
 (segment (start 125.73 88.9) (end 124.46 87.63) (width 0.32) (layer F.Cu) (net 8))
 (segment (start 124.46 87.63) (end 124.46 83.78) (width 0.32) (layer F.Cu) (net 8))
 (via (at 155 74) (size 0.8) (drill 0.4) (layers F.Cu B.Cu) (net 5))
 (segment (start 155 71.5) (end 155 71.5) (width 0.25) (layer B.Cu) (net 5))
 (segment (start 155 71.5) (end 155 74) (width 0.25) (layer B.Cu) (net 5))
 (via (at 155 71.5) (size 0.8) (drill 0.4) (layers F.Cu B.Cu) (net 5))
 (segment (start 163.83 69.85) (end 156.21 69.85) (width 0.3) (layer F.Cu) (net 5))
 (segment (start 170.18 68.54) (end 165.14 68.54) (width 0.3) (layer F.Cu) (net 5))
 (segment (start 165.14 68.54) (end 163.83 69.85) (width 0.3) (layer F.Cu) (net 5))
 (segment (start 156.21 69.85) (end 155.541795 69.818205) (width 0.25) (layer F.Cu) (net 5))
 (segment (start 155.541795 69.818205) (end 153.67 67.31) (width 0.3) (layer F.Cu) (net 5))
 (segment (start 155.541795 69.818205) (end 155.541795 70.958205) (width 0.25) (layer F.Cu) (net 5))
 (segment (start 155.541795 70.958205) (end 155 71.5) (width 0.25) (layer F.Cu) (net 5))
 (segment (start 155 71.5) (end 155 71.5) (width 0.25) (layer B.Cu) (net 5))
 (via (at 155 71.5) (size 0.8) (drill 0.4) (layers F.Cu B.Cu) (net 5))
 (segment (start 155 71.5) (end 155 71.5) (width 0.25) (layer B.Cu) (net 5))
 (via (at 155 71.5) (size 0.8) (drill 0.4) (layers F.Cu B.Cu) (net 5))
 (segment (start 154.395 74.605) (end 155 74) (width 0.25) (layer F.Cu) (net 5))
 (segment (start 153.3398 74.605) (end 154.395 74.605) (width 0.25) (layer F.Cu) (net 5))
 (segment (start 155 74) (end 155 77.664) (width 0.25) (layer F.Cu) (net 5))
 (segment (start 155 77.664) (end 155 77.664) (width 0.25) (layer F.Cu) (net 5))
 (via (at 155 77.664) (size 0.8) (drill 0.4) (layers F.Cu B.Cu) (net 5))
 (segment (start 154.600001 78.063999) (end 154.600001 79.587999) (width 0.25) (layer B.Cu) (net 5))
 (segment (start 155 77.664) (end 154.600001 78.063999) (width 0.25) (layer B.Cu) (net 5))
 (segment (start 154.600001 79.587999) (end 153.416 80.772) (width 0.25) (layer B.Cu) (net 5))
 (segment (start 153.416 80.772) (end 153.416 80.772) (width 0.25) (layer B.Cu) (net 5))
 (via (at 153.416 80.772) (size 0.8) (drill 0.4) (layers F.Cu B.Cu) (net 5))
 (segment (start 153.0183 83.2) (end 152.0698 83.2) (width 0.25) (layer F.Cu) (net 5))
 (segment (start 153.815999 82.402301) (end 153.0183 83.2) (width 0.25) (layer F.Cu) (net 5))
 (segment (start 153.815999 81.171999) (end 153.815999 82.402301) (width 0.25) (layer F.Cu) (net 5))
 (segment (start 153.416 80.772) (end 153.815999 81.171999) (width 0.25) (layer F.Cu) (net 5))
 (segment (start 133.35 104.14) (end 139.7 104.14) (width 0.25) (layer F.Cu) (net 9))
 (segment (start 145.4 83.2) (end 147.6502 83.2) (width 0.25) (layer F.Cu) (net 9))
 (segment (start 143.51 85.09) (end 145.4 83.2) (width 0.25) (layer F.Cu) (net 9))
 (segment (start 143.51 85.09) (end 143.51 103.124) (width 0.25) (layer F.Cu) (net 9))
 (segment (start 142.494 104.14) (end 139.7 104.14) (width 0.25) (layer F.Cu) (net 9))
 (segment (start 143.51 103.124) (end 142.494 104.14) (width 0.25) (layer F.Cu) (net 9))
 (segment (start 139.7 91.44) (end 139.7 87.63) (width 0.25) (layer F.Cu) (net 10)))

